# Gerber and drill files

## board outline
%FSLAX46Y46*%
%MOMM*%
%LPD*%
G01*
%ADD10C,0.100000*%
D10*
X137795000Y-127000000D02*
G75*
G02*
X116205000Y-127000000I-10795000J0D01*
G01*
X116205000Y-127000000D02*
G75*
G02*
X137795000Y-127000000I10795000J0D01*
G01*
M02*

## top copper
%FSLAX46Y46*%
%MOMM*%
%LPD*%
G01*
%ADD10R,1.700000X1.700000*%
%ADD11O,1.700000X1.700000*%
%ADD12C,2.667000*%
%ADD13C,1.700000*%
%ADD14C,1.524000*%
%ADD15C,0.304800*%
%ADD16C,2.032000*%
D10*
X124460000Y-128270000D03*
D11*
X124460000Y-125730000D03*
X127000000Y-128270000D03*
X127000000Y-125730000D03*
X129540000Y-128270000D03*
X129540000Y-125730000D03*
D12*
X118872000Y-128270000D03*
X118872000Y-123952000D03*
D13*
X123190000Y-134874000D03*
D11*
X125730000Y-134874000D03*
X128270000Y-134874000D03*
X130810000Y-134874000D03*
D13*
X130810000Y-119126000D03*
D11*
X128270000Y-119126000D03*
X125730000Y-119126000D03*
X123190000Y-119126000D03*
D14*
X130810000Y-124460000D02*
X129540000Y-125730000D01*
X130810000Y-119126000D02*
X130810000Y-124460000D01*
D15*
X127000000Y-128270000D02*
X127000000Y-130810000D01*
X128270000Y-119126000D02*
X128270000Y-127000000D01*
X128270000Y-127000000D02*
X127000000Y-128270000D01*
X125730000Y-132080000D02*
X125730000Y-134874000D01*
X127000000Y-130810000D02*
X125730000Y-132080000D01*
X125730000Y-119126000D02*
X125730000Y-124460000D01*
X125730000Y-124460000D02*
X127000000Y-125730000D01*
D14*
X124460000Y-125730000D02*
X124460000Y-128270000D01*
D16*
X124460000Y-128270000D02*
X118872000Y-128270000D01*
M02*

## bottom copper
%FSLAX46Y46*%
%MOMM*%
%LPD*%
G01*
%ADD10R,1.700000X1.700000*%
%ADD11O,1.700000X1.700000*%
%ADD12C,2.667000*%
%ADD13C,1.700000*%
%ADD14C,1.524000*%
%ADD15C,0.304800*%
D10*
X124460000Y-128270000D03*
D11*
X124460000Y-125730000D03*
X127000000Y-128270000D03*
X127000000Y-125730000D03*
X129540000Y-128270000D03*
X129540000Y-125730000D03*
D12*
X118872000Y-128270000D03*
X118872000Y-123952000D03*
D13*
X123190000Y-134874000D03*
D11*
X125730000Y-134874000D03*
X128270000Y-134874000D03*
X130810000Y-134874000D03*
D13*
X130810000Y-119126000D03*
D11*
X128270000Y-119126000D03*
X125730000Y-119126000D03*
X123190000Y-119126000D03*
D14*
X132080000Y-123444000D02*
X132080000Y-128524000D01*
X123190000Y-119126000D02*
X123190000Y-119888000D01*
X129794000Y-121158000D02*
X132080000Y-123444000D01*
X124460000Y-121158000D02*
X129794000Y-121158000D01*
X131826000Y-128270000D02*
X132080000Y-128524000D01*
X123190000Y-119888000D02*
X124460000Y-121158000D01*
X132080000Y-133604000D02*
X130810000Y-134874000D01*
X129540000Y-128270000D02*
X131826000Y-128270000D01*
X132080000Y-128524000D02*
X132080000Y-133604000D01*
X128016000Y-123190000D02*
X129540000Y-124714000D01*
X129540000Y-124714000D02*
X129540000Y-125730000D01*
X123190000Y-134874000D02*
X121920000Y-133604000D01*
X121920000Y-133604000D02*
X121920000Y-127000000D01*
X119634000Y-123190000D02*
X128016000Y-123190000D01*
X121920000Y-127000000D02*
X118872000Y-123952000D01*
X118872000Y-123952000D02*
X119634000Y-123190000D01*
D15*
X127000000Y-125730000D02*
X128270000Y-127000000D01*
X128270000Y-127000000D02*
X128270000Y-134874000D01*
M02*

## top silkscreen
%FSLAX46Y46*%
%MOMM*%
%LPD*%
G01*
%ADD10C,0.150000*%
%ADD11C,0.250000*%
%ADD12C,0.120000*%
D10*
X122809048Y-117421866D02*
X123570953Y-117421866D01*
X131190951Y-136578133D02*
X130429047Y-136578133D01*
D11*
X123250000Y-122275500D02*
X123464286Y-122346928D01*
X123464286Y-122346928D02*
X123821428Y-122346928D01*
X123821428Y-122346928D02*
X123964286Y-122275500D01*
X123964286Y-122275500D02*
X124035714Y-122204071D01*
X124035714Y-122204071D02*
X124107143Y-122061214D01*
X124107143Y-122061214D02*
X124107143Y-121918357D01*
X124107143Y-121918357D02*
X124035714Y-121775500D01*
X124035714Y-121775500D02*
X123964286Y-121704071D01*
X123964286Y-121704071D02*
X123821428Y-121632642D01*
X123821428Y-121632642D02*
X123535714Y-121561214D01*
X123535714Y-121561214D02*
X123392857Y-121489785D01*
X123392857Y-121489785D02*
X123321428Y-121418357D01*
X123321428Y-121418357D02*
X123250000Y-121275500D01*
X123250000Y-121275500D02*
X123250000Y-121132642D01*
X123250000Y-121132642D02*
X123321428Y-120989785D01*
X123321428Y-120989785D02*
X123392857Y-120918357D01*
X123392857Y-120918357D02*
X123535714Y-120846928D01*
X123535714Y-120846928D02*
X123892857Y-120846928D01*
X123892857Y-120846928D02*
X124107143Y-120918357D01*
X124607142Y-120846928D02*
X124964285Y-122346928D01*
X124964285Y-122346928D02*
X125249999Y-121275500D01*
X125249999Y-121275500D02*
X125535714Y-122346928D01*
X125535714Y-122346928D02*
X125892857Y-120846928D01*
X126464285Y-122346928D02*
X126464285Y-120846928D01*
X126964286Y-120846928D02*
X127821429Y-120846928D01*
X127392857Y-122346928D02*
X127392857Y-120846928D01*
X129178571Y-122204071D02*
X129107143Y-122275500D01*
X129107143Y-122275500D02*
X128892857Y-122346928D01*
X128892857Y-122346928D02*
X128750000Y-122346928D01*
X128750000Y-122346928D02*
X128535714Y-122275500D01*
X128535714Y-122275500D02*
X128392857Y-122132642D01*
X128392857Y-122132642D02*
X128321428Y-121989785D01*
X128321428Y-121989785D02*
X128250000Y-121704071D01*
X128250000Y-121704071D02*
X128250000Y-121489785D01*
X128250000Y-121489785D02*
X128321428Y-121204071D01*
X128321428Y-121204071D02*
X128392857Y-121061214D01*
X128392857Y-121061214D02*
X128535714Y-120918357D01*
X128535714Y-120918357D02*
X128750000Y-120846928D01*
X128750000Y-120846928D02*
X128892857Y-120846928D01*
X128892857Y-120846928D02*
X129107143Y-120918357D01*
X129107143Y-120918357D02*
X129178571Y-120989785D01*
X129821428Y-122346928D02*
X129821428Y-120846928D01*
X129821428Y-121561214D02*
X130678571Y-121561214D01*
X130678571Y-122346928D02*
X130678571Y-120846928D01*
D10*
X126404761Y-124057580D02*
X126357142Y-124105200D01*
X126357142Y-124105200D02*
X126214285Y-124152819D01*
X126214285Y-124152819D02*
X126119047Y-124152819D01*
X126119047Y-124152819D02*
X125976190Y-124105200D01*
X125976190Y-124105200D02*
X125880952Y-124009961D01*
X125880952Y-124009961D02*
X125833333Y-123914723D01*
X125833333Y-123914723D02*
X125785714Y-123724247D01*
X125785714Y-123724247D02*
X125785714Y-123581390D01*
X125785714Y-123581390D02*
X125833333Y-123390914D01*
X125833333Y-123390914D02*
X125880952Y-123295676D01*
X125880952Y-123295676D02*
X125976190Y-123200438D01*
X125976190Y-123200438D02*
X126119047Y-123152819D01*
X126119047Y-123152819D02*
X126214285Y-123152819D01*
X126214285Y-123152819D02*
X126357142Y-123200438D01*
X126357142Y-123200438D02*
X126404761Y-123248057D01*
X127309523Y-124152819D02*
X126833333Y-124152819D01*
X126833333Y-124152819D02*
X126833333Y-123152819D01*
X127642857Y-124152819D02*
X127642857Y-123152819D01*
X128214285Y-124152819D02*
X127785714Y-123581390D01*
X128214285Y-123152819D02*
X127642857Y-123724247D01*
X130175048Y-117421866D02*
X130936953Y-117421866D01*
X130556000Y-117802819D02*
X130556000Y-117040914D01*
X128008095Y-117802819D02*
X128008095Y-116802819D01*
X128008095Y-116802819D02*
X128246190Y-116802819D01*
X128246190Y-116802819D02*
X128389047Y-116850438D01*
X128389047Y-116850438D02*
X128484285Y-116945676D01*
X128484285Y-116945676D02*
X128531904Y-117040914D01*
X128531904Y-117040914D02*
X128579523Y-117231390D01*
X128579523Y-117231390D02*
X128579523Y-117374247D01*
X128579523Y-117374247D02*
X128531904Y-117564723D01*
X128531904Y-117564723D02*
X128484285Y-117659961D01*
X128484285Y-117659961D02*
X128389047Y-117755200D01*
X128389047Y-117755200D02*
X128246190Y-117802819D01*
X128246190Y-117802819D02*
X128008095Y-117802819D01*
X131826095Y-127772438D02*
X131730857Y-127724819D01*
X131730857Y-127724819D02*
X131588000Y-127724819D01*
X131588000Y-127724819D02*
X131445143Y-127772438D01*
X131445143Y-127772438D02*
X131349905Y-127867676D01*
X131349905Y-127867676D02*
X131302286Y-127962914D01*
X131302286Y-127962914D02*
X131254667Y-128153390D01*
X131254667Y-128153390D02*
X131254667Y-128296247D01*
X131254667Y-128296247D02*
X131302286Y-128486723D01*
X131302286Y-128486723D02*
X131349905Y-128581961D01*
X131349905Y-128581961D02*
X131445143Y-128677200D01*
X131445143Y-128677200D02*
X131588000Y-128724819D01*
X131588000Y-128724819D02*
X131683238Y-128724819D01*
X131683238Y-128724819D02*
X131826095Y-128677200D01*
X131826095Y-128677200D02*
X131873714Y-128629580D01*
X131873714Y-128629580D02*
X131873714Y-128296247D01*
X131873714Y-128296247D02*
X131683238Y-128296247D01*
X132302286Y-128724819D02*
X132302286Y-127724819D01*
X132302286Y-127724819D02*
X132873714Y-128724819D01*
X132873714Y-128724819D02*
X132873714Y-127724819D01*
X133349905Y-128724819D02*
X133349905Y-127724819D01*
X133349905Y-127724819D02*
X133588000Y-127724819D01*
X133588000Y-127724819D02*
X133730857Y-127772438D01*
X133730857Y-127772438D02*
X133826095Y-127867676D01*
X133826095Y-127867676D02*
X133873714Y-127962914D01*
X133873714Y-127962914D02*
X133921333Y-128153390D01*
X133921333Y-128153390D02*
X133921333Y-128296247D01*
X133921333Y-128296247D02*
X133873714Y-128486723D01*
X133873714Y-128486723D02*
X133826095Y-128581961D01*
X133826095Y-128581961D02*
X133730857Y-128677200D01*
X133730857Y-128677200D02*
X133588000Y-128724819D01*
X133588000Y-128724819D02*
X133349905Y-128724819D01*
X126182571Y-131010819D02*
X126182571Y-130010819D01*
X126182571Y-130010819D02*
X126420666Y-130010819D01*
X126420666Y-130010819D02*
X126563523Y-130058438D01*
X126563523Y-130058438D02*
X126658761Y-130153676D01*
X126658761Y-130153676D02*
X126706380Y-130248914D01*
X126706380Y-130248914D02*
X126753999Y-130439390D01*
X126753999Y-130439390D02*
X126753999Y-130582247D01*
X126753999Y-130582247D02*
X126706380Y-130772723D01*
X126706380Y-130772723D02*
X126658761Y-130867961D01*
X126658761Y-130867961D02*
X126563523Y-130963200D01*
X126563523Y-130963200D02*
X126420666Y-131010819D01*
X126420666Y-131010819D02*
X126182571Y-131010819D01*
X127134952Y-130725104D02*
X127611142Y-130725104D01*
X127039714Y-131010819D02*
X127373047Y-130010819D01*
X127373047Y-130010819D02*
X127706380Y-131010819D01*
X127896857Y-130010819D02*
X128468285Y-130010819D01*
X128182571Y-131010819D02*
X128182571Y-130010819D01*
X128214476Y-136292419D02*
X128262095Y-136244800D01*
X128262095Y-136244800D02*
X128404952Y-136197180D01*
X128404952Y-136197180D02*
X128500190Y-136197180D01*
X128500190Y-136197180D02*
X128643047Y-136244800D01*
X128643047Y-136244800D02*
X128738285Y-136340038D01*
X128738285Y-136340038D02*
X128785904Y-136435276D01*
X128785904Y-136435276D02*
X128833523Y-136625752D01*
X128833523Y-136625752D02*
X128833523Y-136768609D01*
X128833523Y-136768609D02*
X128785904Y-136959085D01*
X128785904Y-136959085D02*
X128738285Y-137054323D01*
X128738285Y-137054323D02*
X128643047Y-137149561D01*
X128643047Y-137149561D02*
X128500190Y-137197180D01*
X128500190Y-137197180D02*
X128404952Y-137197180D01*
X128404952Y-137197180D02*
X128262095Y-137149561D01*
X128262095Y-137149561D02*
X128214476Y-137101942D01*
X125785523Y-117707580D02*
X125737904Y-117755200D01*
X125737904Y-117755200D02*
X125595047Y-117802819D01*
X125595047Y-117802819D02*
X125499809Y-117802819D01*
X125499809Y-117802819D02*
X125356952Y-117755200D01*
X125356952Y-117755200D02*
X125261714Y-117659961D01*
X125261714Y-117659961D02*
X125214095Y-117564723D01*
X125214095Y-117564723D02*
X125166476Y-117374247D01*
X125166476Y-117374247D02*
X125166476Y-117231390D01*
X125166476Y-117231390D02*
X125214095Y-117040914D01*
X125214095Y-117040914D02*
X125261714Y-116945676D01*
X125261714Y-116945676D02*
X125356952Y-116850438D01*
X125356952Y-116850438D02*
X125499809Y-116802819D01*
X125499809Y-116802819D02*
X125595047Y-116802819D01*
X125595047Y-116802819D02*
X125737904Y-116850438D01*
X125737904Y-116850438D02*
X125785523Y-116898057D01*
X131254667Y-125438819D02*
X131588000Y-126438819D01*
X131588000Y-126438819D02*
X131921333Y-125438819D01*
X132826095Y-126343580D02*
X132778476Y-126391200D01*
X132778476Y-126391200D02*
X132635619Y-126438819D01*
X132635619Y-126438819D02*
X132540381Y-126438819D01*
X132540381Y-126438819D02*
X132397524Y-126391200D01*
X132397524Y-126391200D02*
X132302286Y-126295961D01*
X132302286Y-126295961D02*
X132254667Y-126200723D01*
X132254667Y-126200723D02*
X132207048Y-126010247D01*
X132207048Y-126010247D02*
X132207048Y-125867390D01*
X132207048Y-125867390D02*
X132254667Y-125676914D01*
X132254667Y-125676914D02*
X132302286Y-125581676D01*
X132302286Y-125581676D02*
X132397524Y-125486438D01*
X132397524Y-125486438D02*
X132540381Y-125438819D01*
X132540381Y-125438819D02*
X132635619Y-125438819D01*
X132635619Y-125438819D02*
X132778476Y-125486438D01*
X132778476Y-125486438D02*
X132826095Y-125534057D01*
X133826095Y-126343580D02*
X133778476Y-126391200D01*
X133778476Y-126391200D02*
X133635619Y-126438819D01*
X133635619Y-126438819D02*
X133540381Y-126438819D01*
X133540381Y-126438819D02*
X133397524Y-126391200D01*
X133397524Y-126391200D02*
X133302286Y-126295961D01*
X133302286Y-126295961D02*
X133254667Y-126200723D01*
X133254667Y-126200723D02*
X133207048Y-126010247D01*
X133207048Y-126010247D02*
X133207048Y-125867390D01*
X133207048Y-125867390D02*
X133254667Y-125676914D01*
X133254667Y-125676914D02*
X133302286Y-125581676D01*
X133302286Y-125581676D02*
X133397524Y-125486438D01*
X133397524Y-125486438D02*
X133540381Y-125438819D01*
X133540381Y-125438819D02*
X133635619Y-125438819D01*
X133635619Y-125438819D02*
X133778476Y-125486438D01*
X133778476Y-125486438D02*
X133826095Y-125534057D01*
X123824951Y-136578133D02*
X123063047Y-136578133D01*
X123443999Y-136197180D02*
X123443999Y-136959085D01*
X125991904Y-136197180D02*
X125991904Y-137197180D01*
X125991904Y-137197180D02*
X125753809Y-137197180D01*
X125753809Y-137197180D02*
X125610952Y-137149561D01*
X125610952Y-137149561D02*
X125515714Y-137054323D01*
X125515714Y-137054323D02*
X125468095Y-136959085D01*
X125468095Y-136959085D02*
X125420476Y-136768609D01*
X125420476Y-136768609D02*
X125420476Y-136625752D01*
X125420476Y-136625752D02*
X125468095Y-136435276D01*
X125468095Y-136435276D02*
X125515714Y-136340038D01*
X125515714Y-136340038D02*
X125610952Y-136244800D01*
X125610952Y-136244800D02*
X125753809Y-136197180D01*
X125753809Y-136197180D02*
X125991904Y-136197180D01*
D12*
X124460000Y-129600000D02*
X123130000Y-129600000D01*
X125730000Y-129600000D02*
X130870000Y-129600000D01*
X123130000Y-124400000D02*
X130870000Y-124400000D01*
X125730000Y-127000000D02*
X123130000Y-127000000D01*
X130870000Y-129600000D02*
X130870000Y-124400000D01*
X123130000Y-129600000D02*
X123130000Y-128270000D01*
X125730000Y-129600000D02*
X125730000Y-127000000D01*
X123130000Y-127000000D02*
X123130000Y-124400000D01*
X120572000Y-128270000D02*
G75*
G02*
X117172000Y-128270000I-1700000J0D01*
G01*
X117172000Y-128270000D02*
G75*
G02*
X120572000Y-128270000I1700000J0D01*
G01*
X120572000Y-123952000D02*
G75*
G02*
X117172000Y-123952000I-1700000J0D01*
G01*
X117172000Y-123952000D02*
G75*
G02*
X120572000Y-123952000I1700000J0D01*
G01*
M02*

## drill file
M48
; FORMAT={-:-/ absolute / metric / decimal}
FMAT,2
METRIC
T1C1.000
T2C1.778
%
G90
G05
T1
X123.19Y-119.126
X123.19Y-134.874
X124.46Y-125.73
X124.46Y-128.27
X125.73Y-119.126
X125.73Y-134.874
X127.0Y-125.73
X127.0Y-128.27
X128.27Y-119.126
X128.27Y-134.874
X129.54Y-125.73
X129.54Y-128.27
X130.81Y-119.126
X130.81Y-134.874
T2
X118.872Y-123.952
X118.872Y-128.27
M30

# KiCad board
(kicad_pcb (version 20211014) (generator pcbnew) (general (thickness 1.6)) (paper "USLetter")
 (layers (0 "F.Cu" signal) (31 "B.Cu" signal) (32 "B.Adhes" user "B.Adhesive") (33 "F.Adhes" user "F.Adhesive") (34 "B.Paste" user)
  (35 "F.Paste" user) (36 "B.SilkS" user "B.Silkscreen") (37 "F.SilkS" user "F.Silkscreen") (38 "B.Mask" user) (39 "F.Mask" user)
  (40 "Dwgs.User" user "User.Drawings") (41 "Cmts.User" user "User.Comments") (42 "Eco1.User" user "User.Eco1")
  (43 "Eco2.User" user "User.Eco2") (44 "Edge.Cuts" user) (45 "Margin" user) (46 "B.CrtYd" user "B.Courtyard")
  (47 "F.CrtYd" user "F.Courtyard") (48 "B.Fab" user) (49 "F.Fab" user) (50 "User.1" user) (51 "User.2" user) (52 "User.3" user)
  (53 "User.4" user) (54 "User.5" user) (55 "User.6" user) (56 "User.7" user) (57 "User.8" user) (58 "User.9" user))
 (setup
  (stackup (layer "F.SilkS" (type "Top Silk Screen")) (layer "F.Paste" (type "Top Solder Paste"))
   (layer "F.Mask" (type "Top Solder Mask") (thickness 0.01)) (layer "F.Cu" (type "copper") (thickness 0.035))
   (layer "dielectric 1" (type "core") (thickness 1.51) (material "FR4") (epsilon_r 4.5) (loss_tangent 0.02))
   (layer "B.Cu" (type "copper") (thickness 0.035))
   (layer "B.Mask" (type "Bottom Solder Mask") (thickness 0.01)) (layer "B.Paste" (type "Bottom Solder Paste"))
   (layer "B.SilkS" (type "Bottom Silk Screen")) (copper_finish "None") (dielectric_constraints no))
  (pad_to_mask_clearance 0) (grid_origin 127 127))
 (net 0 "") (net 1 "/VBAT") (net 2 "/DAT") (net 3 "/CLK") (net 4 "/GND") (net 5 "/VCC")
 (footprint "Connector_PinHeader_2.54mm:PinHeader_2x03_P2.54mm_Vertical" (layer "F.Cu") (at 124.46 128.27 90)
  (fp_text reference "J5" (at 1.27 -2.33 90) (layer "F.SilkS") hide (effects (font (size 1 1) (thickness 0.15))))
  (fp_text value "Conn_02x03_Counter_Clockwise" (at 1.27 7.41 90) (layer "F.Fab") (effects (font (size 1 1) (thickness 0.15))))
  (fp_line (start -1.33 0) (end -1.33 -1.33) (layer "F.SilkS") (width 0.12))
  (fp_line (start -1.33 1.27) (end -1.33 6.41) (layer "F.SilkS") (width 0.12))
  (fp_line (start 3.87 -1.33) (end 3.87 6.41) (layer "F.SilkS") (width 0.12))
  (fp_line (start 1.27 1.27) (end 1.27 -1.33) (layer "F.SilkS") (width 0.12))
  (fp_line (start -1.33 6.41) (end 3.87 6.41) (layer "F.SilkS") (width 0.12))
  (fp_line (start -1.33 -1.33) (end 0 -1.33) (layer "F.SilkS") (width 0.12))
  (fp_line (start -1.33 1.27) (end 1.27 1.27) (layer "F.SilkS") (width 0.12))
  (fp_line (start 1.27 -1.33) (end 3.87 -1.33) (layer "F.SilkS") (width 0.12))
  (pad "1" thru_hole rect (at 0 0 90) (size 1.7 1.7) (drill 1) (layers *.Cu *.Mask) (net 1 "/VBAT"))
  (pad "2" thru_hole oval (at 2.54 0 90) (size 1.7 1.7) (drill 1) (layers *.Cu *.Mask) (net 1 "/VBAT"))
  (pad "3" thru_hole oval (at 0 2.54 90) (size 1.7 1.7) (drill 1) (layers *.Cu *.Mask) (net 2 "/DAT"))
  (pad "4" thru_hole oval (at 2.54 2.54 90) (size 1.7 1.7) (drill 1) (layers *.Cu *.Mask) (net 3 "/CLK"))
  (pad "5" thru_hole oval (at 0 5.08 90) (size 1.7 1.7) (drill 1) (layers *.Cu *.Mask) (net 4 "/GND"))
  (pad "6" thru_hole oval (at 2.54 5.08 90) (size 1.7 1.7) (drill 1) (layers *.Cu *.Mask) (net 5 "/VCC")))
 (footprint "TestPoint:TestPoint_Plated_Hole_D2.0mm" (layer "F.Cu") (at 118.872 128.27)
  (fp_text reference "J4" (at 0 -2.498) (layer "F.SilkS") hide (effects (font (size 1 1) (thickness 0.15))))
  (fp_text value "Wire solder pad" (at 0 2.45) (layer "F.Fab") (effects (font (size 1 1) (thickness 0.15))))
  (fp_circle (center 0 0) (end 0 -1.7) (layer "F.SilkS") (width 0.12) (fill none))
  (pad "1" thru_hole circle (at 0 0) (size 2.667 2.667) (drill 1.778) (layers *.Cu *.Mask) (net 1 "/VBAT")))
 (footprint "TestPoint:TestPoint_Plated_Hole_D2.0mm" (layer "F.Cu") (at 118.872 123.952)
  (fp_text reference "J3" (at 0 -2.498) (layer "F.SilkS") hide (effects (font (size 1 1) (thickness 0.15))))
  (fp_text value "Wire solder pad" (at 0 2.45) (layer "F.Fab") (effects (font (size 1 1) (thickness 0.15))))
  (fp_circle (center 0 0) (end 0 -1.7) (layer "F.SilkS") (width 0.12) (fill none))
  (pad "1" thru_hole circle (at 0 0) (size 2.667 2.667) (drill 1.778) (layers *.Cu *.Mask) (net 5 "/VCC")))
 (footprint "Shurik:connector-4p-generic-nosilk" (layer "F.Cu") (at 123.19 134.874 90)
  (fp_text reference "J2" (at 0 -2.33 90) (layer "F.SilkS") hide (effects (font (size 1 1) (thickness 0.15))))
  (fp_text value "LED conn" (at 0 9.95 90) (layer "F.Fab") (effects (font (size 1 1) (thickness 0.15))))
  (pad "1" thru_hole circle (at 0 0 90) (size 1.7 1.7) (drill 1) (layers *.Cu *.Mask) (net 5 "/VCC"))
  (pad "2" thru_hole oval (at 0 2.54 90) (size 1.7 1.7) (drill 1) (layers *.Cu *.Mask) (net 2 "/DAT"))
  (pad "3" thru_hole oval (at 0 5.08 90) (size 1.7 1.7) (drill 1) (layers *.Cu *.Mask) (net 3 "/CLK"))
  (pad "4" thru_hole oval (at 0 7.62 90) (size 1.7 1.7) (drill 1) (layers *.Cu *.Mask) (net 4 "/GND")))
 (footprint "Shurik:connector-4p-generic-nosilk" (layer "F.Cu") (at 130.81 119.126 -90)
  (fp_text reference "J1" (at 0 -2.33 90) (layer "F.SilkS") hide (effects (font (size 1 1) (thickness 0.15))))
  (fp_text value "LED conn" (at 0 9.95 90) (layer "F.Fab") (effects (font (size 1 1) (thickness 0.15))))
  (pad "1" thru_hole circle (at 0 0 270) (size 1.7 1.7) (drill 1) (layers *.Cu *.Mask) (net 5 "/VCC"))
  (pad "2" thru_hole oval (at 0 2.54 270) (size 1.7 1.7) (drill 1) (layers *.Cu *.Mask) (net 2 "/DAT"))
  (pad "3" thru_hole oval (at 0 5.08 270) (size 1.7 1.7) (drill 1) (layers *.Cu *.Mask) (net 3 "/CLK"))
  (pad "4" thru_hole oval (at 0 7.62 270) (size 1.7 1.7) (drill 1) (layers *.Cu *.Mask) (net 4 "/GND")))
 (gr_arc (start 137.795 127) (mid 127 137.795) (end 116.205 127) (layer "Edge.Cuts") (width 0.1))
 (gr_arc (start 116.205 127) (mid 127 116.205) (end 137.795 127) (layer "Edge.Cuts") (width 0.1))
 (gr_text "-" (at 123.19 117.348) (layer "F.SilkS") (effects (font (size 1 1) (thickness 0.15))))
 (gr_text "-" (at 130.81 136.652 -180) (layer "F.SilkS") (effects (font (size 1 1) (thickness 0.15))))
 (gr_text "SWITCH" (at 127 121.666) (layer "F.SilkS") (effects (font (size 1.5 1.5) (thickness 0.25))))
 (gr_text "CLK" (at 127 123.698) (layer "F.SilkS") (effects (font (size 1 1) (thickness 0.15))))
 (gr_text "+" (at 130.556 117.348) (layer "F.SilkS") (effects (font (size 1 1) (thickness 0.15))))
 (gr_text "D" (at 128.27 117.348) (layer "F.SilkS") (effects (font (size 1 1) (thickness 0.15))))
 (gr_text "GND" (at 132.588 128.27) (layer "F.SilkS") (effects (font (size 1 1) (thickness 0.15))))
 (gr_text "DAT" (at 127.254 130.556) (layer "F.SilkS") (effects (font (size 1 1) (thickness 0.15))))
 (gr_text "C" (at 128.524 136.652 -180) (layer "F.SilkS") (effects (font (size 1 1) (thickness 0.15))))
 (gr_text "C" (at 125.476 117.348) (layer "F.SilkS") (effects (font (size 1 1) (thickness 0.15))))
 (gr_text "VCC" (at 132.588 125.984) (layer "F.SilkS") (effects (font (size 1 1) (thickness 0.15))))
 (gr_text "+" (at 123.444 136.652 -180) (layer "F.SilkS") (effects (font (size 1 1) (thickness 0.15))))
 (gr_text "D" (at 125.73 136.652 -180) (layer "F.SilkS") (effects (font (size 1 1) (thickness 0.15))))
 (segment (start 132.08 123.444) (end 132.08 128.524) (width 1.524) (layer "B.Cu") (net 4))
 (segment (start 123.19 119.126) (end 123.19 119.888) (width 1.524) (layer "B.Cu") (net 4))
 (segment (start 129.794 121.158) (end 132.08 123.444) (width 1.524) (layer "B.Cu") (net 4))
 (segment (start 124.46 121.158) (end 129.794 121.158) (width 1.524) (layer "B.Cu") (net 4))
 (segment (start 131.826 128.27) (end 132.08 128.524) (width 1.524) (layer "B.Cu") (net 4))
 (segment (start 123.19 119.888) (end 124.46 121.158) (width 1.524) (layer "B.Cu") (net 4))
 (segment (start 132.08 133.604) (end 130.81 134.874) (width 1.524) (layer "B.Cu") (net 4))
 (segment (start 129.54 128.27) (end 131.826 128.27) (width 1.524) (layer "B.Cu") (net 4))
 (segment (start 132.08 128.524) (end 132.08 133.604) (width 1.524) (layer "B.Cu") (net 4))
 (segment (start 130.81 124.46) (end 129.54 125.73) (width 1.524) (layer "F.Cu") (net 5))
 (segment (start 130.81 119.126) (end 130.81 124.46) (width 1.524) (layer "F.Cu") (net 5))
 (segment (start 128.016 123.19) (end 129.54 124.714) (width 1.524) (layer "B.Cu") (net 5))
 (segment (start 129.54 124.714) (end 129.54 125.73) (width 1.524) (layer "B.Cu") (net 5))
 (segment (start 123.19 134.874) (end 121.92 133.604) (width 1.524) (layer "B.Cu") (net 5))
 (segment (start 121.92 133.604) (end 121.92 127) (width 1.524) (layer "B.Cu") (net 5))
 (segment (start 119.634 123.19) (end 128.016 123.19) (width 1.524) (layer "B.Cu") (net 5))
 (segment (start 121.92 127) (end 118.872 123.952) (width 1.524) (layer "B.Cu") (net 5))
 (segment (start 118.872 123.952) (end 119.634 123.19) (width 1.524) (layer "B.Cu") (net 5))
 (segment (start 127 128.27) (end 127 130.81) (width 0.3048) (layer "F.Cu") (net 2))
 (segment (start 128.27 119.126) (end 128.27 127) (width 0.3048) (layer "F.Cu") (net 2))
 (segment (start 128.27 127) (end 127 128.27) (width 0.3048) (layer "F.Cu") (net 2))
 (segment (start 125.73 132.08) (end 125.73 134.874) (width 0.3048) (layer "F.Cu") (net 2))
 (segment (start 127 130.81) (end 125.73 132.08) (width 0.3048) (layer "F.Cu") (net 2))
 (segment (start 125.73 119.126) (end 125.73 124.46) (width 0.3048) (layer "F.Cu") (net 3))
 (segment (start 125.73 124.46) (end 127 125.73) (width 0.3048) (layer "F.Cu") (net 3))
 (segment (start 127 125.73) (end 128.27 127) (width 0.3048) (layer "B.Cu") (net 3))
 (segment (start 128.27 127) (end 128.27 134.874) (width 0.3048) (layer "B.Cu") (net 3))
 (segment (start 124.46 125.73) (end 124.46 128.27) (width 1.524) (layer "F.Cu") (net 1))
 (segment (start 124.46 128.27) (end 118.872 128.27) (width 2.032) (layer "F.Cu") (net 1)))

